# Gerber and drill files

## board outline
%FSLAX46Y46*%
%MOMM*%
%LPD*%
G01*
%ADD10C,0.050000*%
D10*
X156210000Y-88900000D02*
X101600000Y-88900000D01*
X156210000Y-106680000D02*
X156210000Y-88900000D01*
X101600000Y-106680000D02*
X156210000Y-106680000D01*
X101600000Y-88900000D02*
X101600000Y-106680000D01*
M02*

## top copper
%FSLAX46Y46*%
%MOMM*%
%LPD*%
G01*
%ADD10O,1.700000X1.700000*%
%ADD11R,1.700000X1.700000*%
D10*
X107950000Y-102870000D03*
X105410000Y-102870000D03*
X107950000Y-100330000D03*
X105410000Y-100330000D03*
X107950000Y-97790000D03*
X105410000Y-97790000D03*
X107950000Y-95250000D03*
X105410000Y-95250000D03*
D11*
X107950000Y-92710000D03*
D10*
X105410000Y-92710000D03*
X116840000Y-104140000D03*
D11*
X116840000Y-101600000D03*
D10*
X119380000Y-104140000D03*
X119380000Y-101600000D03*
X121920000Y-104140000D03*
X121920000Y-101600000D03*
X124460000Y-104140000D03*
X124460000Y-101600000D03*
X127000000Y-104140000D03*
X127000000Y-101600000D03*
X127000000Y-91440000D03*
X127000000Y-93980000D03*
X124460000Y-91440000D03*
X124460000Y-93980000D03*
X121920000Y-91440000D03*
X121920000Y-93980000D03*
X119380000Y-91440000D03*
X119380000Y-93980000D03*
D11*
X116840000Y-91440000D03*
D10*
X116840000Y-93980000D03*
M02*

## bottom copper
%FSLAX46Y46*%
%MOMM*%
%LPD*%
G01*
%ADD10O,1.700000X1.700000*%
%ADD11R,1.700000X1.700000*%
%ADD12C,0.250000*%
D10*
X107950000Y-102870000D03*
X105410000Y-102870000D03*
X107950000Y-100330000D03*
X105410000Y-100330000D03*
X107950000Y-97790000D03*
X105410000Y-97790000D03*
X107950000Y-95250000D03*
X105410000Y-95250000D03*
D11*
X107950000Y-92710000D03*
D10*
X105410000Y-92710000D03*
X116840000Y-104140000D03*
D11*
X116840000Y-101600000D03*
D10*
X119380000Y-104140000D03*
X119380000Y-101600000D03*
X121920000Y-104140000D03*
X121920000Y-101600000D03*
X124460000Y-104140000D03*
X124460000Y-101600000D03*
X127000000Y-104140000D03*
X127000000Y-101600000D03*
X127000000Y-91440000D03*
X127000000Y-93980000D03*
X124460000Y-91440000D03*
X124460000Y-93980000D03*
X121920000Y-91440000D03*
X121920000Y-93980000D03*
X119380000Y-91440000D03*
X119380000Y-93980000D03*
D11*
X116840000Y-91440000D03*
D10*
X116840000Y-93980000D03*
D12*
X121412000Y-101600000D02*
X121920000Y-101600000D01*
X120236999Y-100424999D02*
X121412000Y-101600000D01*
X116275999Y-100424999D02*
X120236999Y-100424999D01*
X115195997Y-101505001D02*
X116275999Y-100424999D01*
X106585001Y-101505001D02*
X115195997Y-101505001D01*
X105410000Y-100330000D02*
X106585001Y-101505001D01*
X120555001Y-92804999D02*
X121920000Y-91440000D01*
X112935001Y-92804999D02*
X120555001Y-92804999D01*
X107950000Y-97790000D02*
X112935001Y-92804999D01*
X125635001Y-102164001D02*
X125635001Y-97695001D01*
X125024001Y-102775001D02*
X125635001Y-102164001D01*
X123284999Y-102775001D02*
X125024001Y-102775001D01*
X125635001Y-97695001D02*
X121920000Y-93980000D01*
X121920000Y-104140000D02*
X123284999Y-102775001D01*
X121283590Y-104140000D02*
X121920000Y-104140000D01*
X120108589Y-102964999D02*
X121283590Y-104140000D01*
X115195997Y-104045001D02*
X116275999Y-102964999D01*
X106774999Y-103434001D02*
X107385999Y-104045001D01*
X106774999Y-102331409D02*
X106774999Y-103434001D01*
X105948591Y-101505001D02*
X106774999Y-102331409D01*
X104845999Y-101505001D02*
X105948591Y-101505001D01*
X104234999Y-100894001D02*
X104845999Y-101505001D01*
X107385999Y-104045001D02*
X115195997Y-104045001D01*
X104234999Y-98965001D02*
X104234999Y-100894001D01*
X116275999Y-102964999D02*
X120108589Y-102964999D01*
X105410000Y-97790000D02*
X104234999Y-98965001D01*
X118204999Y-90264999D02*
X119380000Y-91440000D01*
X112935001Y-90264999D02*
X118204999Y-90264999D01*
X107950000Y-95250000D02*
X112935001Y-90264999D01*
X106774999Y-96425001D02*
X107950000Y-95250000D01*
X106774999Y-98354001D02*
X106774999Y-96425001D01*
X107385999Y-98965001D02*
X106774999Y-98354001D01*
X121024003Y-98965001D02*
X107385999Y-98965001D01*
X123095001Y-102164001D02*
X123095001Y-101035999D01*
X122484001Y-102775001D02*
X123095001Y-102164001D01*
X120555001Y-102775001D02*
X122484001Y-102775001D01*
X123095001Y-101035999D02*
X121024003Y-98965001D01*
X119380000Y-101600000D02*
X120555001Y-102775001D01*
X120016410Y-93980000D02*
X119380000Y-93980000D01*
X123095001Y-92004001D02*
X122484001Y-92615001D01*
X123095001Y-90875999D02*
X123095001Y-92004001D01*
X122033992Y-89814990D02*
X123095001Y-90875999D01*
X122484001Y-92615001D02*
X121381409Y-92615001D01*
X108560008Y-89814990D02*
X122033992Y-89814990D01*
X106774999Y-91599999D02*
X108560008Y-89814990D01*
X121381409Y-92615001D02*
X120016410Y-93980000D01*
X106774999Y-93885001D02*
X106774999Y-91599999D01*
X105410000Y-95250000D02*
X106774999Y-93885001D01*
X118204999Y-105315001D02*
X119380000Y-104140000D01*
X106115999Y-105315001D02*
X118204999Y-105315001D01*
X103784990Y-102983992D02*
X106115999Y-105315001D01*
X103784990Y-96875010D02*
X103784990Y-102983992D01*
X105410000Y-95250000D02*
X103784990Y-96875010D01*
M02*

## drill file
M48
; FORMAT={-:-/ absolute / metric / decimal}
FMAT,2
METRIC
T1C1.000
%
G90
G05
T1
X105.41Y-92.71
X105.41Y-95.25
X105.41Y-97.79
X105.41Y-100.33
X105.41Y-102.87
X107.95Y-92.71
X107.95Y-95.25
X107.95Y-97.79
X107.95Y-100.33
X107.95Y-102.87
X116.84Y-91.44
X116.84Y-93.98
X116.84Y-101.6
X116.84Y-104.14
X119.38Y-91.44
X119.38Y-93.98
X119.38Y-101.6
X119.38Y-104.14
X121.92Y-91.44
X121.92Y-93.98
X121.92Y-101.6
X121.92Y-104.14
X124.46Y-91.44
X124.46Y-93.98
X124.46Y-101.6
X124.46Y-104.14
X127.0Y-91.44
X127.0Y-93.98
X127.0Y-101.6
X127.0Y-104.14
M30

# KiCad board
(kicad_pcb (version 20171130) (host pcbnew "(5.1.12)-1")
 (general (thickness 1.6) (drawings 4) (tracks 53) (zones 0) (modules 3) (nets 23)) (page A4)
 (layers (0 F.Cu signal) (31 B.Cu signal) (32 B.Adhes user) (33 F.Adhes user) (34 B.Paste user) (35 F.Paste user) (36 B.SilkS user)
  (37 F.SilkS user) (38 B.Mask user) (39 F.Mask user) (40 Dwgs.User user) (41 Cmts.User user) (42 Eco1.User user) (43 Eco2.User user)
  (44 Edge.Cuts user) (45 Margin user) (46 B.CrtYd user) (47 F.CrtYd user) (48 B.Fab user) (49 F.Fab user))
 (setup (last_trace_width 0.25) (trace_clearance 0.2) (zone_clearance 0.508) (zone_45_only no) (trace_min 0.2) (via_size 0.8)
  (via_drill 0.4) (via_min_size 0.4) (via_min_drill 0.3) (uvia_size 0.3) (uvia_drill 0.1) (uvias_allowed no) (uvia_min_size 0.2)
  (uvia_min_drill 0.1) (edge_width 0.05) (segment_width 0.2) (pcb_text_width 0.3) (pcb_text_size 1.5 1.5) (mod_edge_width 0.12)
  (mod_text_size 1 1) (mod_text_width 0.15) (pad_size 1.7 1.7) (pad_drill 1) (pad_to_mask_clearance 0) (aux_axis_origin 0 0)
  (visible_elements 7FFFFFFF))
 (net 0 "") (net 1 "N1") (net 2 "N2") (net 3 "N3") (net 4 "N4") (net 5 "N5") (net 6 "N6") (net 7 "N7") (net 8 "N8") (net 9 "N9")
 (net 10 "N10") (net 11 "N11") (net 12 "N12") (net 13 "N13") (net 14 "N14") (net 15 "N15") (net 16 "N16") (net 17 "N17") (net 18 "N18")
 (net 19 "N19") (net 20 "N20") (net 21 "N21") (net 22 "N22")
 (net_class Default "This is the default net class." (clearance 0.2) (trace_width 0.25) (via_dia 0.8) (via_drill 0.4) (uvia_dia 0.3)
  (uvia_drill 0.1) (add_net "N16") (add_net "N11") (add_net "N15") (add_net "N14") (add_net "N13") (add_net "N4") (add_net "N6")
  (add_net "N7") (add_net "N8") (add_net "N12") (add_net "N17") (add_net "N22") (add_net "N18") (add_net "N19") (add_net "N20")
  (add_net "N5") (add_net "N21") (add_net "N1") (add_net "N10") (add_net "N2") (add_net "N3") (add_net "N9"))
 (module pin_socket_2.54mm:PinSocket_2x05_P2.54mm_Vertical (layer B.Cu) (at 107.95 102.87)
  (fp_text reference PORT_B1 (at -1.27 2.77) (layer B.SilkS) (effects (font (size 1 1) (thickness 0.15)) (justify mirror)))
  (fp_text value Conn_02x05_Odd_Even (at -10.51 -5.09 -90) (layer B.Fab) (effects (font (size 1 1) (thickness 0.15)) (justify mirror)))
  (pad 1 thru_hole oval (at 0 0) (size 1.7 1.7) (drill 1) (layers *.Cu *.Mask) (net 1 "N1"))
  (pad 2 thru_hole oval (at -2.54 0) (size 1.7 1.7) (drill 1) (layers *.Cu *.Mask) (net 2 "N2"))
  (pad 3 thru_hole oval (at 0 -2.54) (size 1.7 1.7) (drill 1) (layers *.Cu *.Mask) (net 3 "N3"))
  (pad 4 thru_hole oval (at -2.54 -2.54) (size 1.7 1.7) (drill 1) (layers *.Cu *.Mask) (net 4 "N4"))
  (pad 5 thru_hole oval (at 0 -5.08) (size 1.7 1.7) (drill 1) (layers *.Cu *.Mask) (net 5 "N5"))
  (pad 6 thru_hole oval (at -2.54 -5.08) (size 1.7 1.7) (drill 1) (layers *.Cu *.Mask) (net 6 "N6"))
  (pad 7 thru_hole oval (at 0 -7.62) (size 1.7 1.7) (drill 1) (layers *.Cu *.Mask) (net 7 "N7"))
  (pad 8 thru_hole oval (at -2.54 -7.62) (size 1.7 1.7) (drill 1) (layers *.Cu *.Mask) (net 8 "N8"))
  (pad 9 thru_hole rect (at 0 -10.16) (size 1.7 1.7) (drill 1) (layers *.Cu *.Mask) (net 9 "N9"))
  (pad 10 thru_hole oval (at -2.54 -10.16) (size 1.7 1.7) (drill 1) (layers *.Cu *.Mask) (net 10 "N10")))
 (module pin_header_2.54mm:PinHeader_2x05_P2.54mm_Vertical (layer F.Cu) (at 127 101.6 270)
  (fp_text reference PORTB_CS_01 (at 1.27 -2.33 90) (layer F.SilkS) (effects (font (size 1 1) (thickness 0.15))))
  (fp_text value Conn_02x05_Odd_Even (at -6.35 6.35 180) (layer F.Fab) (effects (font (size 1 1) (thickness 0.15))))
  (pad 10 thru_hole oval (at 2.54 10.16 270) (size 1.7 1.7) (drill 1) (layers *.Cu *.Mask) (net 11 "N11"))
  (pad 9 thru_hole rect (at 0 10.16 270) (size 1.7 1.7) (drill 1) (layers *.Cu *.Mask) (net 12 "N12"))
  (pad 8 thru_hole oval (at 2.54 7.62 270) (size 1.7 1.7) (drill 1) (layers *.Cu *.Mask) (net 8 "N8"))
  (pad 7 thru_hole oval (at 0 7.62 270) (size 1.7 1.7) (drill 1) (layers *.Cu *.Mask) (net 7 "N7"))
  (pad 6 thru_hole oval (at 2.54 5.08 270) (size 1.7 1.7) (drill 1) (layers *.Cu *.Mask) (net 6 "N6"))
  (pad 5 thru_hole oval (at 0 5.08 270) (size 1.7 1.7) (drill 1) (layers *.Cu *.Mask) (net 4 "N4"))
  (pad 4 thru_hole oval (at 2.54 2.54 270) (size 1.7 1.7) (drill 1) (layers *.Cu *.Mask) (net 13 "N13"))
  (pad 3 thru_hole oval (at 0 2.54 270) (size 1.7 1.7) (drill 1) (layers *.Cu *.Mask) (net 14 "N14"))
  (pad 2 thru_hole oval (at 2.54 0 270) (size 1.7 1.7) (drill 1) (layers *.Cu *.Mask) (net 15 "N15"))
  (pad 1 thru_hole oval (at 0 0 270) (size 1.7 1.7) (drill 1) (layers *.Cu *.Mask) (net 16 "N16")))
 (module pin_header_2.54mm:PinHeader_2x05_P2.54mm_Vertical (layer F.Cu) (at 127 91.44 270)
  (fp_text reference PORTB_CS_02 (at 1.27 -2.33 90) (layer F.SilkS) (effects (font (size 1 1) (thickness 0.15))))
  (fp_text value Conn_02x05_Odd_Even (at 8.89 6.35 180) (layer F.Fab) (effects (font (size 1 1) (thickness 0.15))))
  (pad 1 thru_hole oval (at 0 0 270) (size 1.7 1.7) (drill 1) (layers *.Cu *.Mask) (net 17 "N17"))
  (pad 2 thru_hole oval (at 2.54 0 270) (size 1.7 1.7) (drill 1) (layers *.Cu *.Mask) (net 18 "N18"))
  (pad 3 thru_hole oval (at 0 2.54 270) (size 1.7 1.7) (drill 1) (layers *.Cu *.Mask) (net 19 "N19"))
  (pad 4 thru_hole oval (at 2.54 2.54 270) (size 1.7 1.7) (drill 1) (layers *.Cu *.Mask) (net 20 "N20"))
  (pad 5 thru_hole oval (at 0 5.08 270) (size 1.7 1.7) (drill 1) (layers *.Cu *.Mask) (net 5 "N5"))
  (pad 6 thru_hole oval (at 2.54 5.08 270) (size 1.7 1.7) (drill 1) (layers *.Cu *.Mask) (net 6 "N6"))
  (pad 7 thru_hole oval (at 0 7.62 270) (size 1.7 1.7) (drill 1) (layers *.Cu *.Mask) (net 7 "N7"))
  (pad 8 thru_hole oval (at 2.54 7.62 270) (size 1.7 1.7) (drill 1) (layers *.Cu *.Mask) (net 8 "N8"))
  (pad 9 thru_hole rect (at 0 10.16 270) (size 1.7 1.7) (drill 1) (layers *.Cu *.Mask) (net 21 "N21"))
  (pad 10 thru_hole oval (at 2.54 10.16 270) (size 1.7 1.7) (drill 1) (layers *.Cu *.Mask) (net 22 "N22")))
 (gr_line (start 156.21 88.9) (end 101.6 88.9) (layer Edge.Cuts) (width 0.05))
 (gr_line (start 156.21 106.68) (end 156.21 88.9) (layer Edge.Cuts) (width 0.05))
 (gr_line (start 101.6 106.68) (end 156.21 106.68) (layer Edge.Cuts) (width 0.05))
 (gr_line (start 101.6 88.9) (end 101.6 106.68) (layer Edge.Cuts) (width 0.05))
 (segment (start 121.412 101.6) (end 121.92 101.6) (width 0.25) (layer B.Cu) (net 4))
 (segment (start 120.236999 100.424999) (end 121.412 101.6) (width 0.25) (layer B.Cu) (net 4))
 (segment (start 116.275999 100.424999) (end 120.236999 100.424999) (width 0.25) (layer B.Cu) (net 4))
 (segment (start 115.195997 101.505001) (end 116.275999 100.424999) (width 0.25) (layer B.Cu) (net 4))
 (segment (start 106.585001 101.505001) (end 115.195997 101.505001) (width 0.25) (layer B.Cu) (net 4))
 (segment (start 105.41 100.33) (end 106.585001 101.505001) (width 0.25) (layer B.Cu) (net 4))
 (segment (start 120.555001 92.804999) (end 121.92 91.44) (width 0.25) (layer B.Cu) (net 5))
 (segment (start 112.935001 92.804999) (end 120.555001 92.804999) (width 0.25) (layer B.Cu) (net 5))
 (segment (start 107.95 97.79) (end 112.935001 92.804999) (width 0.25) (layer B.Cu) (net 5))
 (segment (start 125.635001 102.164001) (end 125.635001 97.695001) (width 0.25) (layer B.Cu) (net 6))
 (segment (start 125.024001 102.775001) (end 125.635001 102.164001) (width 0.25) (layer B.Cu) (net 6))
 (segment (start 123.284999 102.775001) (end 125.024001 102.775001) (width 0.25) (layer B.Cu) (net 6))
 (segment (start 125.635001 97.695001) (end 121.92 93.98) (width 0.25) (layer B.Cu) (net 6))
 (segment (start 121.92 104.14) (end 123.284999 102.775001) (width 0.25) (layer B.Cu) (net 6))
 (segment (start 121.28359 104.14) (end 121.92 104.14) (width 0.25) (layer B.Cu) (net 6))
 (segment (start 120.108589 102.964999) (end 121.28359 104.14) (width 0.25) (layer B.Cu) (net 6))
 (segment (start 115.195997 104.045001) (end 116.275999 102.964999) (width 0.25) (layer B.Cu) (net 6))
 (segment (start 106.774999 103.434001) (end 107.385999 104.045001) (width 0.25) (layer B.Cu) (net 6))
 (segment (start 106.774999 102.331409) (end 106.774999 103.434001) (width 0.25) (layer B.Cu) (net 6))
 (segment (start 105.948591 101.505001) (end 106.774999 102.331409) (width 0.25) (layer B.Cu) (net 6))
 (segment (start 104.845999 101.505001) (end 105.948591 101.505001) (width 0.25) (layer B.Cu) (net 6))
 (segment (start 104.234999 100.894001) (end 104.845999 101.505001) (width 0.25) (layer B.Cu) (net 6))
 (segment (start 107.385999 104.045001) (end 115.195997 104.045001) (width 0.25) (layer B.Cu) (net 6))
 (segment (start 104.234999 98.965001) (end 104.234999 100.894001) (width 0.25) (layer B.Cu) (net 6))
 (segment (start 116.275999 102.964999) (end 120.108589 102.964999) (width 0.25) (layer B.Cu) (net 6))
 (segment (start 105.41 97.79) (end 104.234999 98.965001) (width 0.25) (layer B.Cu) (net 6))
 (segment (start 118.204999 90.264999) (end 119.38 91.44) (width 0.25) (layer B.Cu) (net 7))
 (segment (start 112.935001 90.264999) (end 118.204999 90.264999) (width 0.25) (layer B.Cu) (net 7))
 (segment (start 107.95 95.25) (end 112.935001 90.264999) (width 0.25) (layer B.Cu) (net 7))
 (segment (start 106.774999 96.425001) (end 107.95 95.25) (width 0.25) (layer B.Cu) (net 7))
 (segment (start 106.774999 98.354001) (end 106.774999 96.425001) (width 0.25) (layer B.Cu) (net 7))
 (segment (start 107.385999 98.965001) (end 106.774999 98.354001) (width 0.25) (layer B.Cu) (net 7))
 (segment (start 121.024003 98.965001) (end 107.385999 98.965001) (width 0.25) (layer B.Cu) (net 7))
 (segment (start 123.095001 102.164001) (end 123.095001 101.035999) (width 0.25) (layer B.Cu) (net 7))
 (segment (start 122.484001 102.775001) (end 123.095001 102.164001) (width 0.25) (layer B.Cu) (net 7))
 (segment (start 120.555001 102.775001) (end 122.484001 102.775001) (width 0.25) (layer B.Cu) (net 7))
 (segment (start 123.095001 101.035999) (end 121.024003 98.965001) (width 0.25) (layer B.Cu) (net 7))
 (segment (start 119.38 101.6) (end 120.555001 102.775001) (width 0.25) (layer B.Cu) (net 7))
 (segment (start 120.01641 93.98) (end 119.38 93.98) (width 0.25) (layer B.Cu) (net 8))
 (segment (start 123.095001 92.004001) (end 122.484001 92.615001) (width 0.25) (layer B.Cu) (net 8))
 (segment (start 123.095001 90.875999) (end 123.095001 92.004001) (width 0.25) (layer B.Cu) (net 8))
 (segment (start 122.033992 89.81499) (end 123.095001 90.875999) (width 0.25) (layer B.Cu) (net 8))
 (segment (start 122.484001 92.615001) (end 121.381409 92.615001) (width 0.25) (layer B.Cu) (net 8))
 (segment (start 108.560008 89.81499) (end 122.033992 89.81499) (width 0.25) (layer B.Cu) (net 8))
 (segment (start 106.774999 91.599999) (end 108.560008 89.81499) (width 0.25) (layer B.Cu) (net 8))
 (segment (start 121.381409 92.615001) (end 120.01641 93.98) (width 0.25) (layer B.Cu) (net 8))
 (segment (start 106.774999 93.885001) (end 106.774999 91.599999) (width 0.25) (layer B.Cu) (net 8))
 (segment (start 105.41 95.25) (end 106.774999 93.885001) (width 0.25) (layer B.Cu) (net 8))
 (segment (start 118.204999 105.315001) (end 119.38 104.14) (width 0.25) (layer B.Cu) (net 8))
 (segment (start 106.115999 105.315001) (end 118.204999 105.315001) (width 0.25) (layer B.Cu) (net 8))
 (segment (start 103.78499 102.983992) (end 106.115999 105.315001) (width 0.25) (layer B.Cu) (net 8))
 (segment (start 103.78499 96.87501) (end 103.78499 102.983992) (width 0.25) (layer B.Cu) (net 8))
 (segment (start 105.41 95.25) (end 103.78499 96.87501) (width 0.25) (layer B.Cu) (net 8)))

